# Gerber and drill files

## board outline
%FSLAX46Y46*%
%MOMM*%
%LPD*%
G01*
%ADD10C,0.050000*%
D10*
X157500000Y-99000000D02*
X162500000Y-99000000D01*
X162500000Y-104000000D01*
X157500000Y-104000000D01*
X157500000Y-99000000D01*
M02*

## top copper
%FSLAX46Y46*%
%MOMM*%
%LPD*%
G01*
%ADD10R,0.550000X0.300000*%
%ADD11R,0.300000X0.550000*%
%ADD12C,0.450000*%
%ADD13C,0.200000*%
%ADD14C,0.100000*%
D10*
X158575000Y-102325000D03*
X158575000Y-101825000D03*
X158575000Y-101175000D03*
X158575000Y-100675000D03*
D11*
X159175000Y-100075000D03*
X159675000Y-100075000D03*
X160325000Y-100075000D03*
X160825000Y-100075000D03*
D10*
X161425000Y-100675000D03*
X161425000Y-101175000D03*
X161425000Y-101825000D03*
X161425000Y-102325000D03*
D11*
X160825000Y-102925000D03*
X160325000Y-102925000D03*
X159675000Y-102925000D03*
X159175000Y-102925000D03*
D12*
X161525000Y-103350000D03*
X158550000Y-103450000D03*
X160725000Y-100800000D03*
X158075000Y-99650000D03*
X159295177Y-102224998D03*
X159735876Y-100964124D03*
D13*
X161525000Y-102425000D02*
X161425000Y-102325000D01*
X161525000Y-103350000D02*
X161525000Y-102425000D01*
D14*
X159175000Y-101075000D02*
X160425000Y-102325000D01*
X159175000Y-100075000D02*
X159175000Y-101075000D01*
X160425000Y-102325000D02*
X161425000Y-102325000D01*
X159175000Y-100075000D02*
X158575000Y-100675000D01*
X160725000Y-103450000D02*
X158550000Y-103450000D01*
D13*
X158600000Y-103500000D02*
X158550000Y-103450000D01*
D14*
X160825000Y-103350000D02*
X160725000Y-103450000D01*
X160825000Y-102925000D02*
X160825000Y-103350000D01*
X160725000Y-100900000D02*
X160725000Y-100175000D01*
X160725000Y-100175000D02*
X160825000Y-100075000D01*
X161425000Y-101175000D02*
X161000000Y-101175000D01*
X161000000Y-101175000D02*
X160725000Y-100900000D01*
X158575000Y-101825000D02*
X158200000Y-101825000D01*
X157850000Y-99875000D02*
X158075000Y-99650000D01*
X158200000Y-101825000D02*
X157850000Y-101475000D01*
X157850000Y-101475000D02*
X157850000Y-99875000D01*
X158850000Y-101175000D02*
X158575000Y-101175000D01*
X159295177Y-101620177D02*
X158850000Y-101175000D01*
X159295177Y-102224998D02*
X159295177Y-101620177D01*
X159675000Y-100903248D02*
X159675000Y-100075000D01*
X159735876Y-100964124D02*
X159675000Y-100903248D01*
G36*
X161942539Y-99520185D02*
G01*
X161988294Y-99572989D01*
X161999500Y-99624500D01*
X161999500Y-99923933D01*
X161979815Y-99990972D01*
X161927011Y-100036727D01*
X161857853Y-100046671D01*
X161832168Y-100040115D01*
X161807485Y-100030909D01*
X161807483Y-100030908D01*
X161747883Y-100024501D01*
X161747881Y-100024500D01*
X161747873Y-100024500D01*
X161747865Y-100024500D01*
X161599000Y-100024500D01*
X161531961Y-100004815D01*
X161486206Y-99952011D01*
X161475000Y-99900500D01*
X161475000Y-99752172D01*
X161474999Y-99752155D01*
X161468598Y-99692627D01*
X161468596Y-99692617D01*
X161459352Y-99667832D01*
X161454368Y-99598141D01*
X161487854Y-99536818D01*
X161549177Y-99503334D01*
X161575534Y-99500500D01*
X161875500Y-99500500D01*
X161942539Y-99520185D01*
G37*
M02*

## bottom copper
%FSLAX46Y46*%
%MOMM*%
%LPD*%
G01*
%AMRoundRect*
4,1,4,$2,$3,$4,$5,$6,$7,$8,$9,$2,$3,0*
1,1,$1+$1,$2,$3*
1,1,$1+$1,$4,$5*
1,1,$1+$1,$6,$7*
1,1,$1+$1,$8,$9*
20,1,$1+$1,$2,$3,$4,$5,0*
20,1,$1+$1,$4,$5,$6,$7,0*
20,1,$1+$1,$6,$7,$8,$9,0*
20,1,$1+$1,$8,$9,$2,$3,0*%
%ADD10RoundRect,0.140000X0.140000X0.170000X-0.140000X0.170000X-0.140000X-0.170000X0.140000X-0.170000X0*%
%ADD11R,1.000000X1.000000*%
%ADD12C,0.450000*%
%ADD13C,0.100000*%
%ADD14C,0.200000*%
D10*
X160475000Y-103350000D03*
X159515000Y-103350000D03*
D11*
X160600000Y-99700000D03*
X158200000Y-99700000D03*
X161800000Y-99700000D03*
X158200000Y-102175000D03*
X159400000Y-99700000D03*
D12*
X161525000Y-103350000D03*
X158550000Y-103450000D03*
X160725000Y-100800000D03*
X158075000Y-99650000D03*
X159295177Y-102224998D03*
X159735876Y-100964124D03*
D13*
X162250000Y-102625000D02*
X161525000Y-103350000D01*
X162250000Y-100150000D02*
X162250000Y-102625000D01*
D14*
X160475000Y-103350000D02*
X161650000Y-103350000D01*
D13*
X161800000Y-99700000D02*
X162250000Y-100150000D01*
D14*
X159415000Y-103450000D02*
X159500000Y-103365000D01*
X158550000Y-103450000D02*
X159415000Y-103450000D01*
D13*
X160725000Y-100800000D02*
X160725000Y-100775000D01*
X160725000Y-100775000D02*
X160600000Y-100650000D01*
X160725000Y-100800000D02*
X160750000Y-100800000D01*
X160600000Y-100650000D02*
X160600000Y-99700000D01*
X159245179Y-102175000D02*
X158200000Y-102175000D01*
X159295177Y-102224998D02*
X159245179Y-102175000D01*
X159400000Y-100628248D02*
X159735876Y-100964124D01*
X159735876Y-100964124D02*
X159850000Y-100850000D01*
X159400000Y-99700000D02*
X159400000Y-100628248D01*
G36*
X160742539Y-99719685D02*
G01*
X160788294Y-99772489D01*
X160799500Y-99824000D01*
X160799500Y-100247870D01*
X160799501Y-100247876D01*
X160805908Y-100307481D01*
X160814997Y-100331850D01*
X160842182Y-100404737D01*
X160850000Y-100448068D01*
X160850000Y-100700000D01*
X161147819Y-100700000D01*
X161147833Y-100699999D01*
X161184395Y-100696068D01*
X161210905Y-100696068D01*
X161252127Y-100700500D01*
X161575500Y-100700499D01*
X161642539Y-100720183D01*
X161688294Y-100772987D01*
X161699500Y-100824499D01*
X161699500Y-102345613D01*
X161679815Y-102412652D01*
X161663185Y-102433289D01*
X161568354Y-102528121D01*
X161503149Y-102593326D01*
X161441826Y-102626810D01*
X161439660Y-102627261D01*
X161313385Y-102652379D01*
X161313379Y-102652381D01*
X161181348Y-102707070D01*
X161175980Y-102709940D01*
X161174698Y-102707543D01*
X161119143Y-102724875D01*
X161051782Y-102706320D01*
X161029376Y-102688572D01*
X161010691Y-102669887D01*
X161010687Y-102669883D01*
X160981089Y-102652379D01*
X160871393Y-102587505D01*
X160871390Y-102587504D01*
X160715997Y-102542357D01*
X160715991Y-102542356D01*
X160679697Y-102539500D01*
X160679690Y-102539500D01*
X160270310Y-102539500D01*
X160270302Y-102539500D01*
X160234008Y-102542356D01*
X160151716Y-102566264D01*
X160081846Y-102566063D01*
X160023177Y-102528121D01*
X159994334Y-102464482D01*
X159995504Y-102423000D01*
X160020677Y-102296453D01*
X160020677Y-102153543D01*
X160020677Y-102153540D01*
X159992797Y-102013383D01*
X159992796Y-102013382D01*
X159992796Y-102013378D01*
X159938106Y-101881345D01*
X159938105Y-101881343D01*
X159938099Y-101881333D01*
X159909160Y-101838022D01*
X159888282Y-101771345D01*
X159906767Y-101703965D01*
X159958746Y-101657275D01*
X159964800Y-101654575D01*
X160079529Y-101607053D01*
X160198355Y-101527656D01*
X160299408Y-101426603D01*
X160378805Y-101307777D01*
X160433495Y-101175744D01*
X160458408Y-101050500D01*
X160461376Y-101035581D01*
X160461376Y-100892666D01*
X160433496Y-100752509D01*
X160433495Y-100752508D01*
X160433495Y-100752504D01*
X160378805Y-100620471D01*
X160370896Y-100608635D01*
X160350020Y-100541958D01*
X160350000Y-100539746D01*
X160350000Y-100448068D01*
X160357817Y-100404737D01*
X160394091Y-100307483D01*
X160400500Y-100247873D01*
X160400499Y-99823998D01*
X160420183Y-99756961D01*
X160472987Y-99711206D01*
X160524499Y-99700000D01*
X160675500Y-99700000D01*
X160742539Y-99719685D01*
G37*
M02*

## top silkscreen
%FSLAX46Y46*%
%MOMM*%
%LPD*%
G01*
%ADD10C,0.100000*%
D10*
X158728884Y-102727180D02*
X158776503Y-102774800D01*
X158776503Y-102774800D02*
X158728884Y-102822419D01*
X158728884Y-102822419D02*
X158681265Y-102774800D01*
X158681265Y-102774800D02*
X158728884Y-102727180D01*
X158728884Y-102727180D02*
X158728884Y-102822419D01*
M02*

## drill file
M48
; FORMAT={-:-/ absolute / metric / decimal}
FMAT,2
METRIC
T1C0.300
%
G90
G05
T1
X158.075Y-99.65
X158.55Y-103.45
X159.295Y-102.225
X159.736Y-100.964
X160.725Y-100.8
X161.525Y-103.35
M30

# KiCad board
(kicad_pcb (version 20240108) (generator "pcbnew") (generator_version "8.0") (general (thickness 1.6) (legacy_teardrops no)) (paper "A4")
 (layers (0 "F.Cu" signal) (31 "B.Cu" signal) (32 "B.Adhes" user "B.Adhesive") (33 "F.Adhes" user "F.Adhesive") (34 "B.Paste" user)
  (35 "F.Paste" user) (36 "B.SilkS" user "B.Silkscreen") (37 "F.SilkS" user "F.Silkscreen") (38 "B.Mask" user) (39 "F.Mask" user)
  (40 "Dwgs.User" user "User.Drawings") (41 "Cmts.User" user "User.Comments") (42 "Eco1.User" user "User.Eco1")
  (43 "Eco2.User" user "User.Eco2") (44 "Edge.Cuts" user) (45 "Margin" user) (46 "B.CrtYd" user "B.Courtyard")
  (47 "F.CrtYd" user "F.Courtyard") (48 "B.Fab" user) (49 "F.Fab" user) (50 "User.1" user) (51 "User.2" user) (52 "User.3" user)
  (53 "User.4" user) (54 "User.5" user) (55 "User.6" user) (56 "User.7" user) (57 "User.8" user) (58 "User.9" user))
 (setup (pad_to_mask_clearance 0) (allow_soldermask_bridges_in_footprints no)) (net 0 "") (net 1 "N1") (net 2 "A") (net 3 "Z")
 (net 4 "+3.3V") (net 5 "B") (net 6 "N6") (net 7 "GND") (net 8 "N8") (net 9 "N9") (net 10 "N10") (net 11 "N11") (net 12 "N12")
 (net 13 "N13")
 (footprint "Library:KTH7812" (layer "F.Cu") (at 158.5 103)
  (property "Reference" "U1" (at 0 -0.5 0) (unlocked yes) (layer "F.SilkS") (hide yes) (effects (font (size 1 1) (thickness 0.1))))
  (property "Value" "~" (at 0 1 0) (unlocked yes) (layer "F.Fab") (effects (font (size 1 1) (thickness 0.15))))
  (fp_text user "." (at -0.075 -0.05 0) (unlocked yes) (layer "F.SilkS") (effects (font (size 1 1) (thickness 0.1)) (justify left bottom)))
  (pad "1" smd rect (at 0.075 -0.675 180) (size 0.55 0.3) (layers "F.Cu" "F.Paste" "F.Mask") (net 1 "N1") (thermal_bridge_angle 45))
  (pad "2" smd rect (at 0.075 -1.175 180) (size 0.55 0.3) (layers "F.Cu" "F.Paste" "F.Mask") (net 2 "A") (thermal_bridge_angle 45))
  (pad "3" smd rect (at 0.075 -1.825 180) (size 0.55 0.3) (layers "F.Cu" "F.Paste" "F.Mask") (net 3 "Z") (thermal_bridge_angle 45))
  (pad "4" smd rect (at 0.075 -2.325 180) (size 0.55 0.3) (layers "F.Cu" "F.Paste" "F.Mask") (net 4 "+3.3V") (thermal_bridge_angle 45))
  (pad "5" smd rect (at 0.675 -2.925 90) (size 0.55 0.3) (layers "F.Cu" "F.Paste" "F.Mask") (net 4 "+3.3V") (thermal_bridge_angle 45))
  (pad "6" smd rect (at 1.175 -2.925 90) (size 0.55 0.3) (layers "F.Cu" "F.Paste" "F.Mask") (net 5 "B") (thermal_bridge_angle 45))
  (pad "7" smd rect (at 1.825 -2.925 90) (size 0.55 0.3) (layers "F.Cu" "F.Paste" "F.Mask") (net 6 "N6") (thermal_bridge_angle 45))
  (pad "8" smd rect (at 2.325 -2.925 90) (size 0.55 0.3) (layers "F.Cu" "F.Paste" "F.Mask") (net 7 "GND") (thermal_bridge_angle 45))
  (pad "9" smd rect (at 2.925 -2.325) (size 0.55 0.3) (layers "F.Cu" "F.Paste" "F.Mask") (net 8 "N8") (thermal_bridge_angle 45))
  (pad "10" smd rect (at 2.925 -1.825) (size 0.55 0.3) (layers "F.Cu" "F.Paste" "F.Mask") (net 7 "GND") (thermal_bridge_angle 45))
  (pad "11" smd rect (at 2.925 -1.175) (size 0.55 0.3) (layers "F.Cu" "F.Paste" "F.Mask") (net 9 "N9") (thermal_bridge_angle 45))
  (pad "12" smd rect (at 2.925 -0.675) (size 0.55 0.3) (layers "F.Cu" "F.Paste" "F.Mask") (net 4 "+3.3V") (thermal_bridge_angle 45))
  (pad "13" smd rect (at 2.325 -0.075 270) (size 0.55 0.3) (layers "F.Cu" "F.Paste" "F.Mask") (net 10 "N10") (thermal_bridge_angle 45))
  (pad "14" smd rect (at 1.825 -0.075 270) (size 0.55 0.3) (layers "F.Cu" "F.Paste" "F.Mask") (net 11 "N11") (thermal_bridge_angle 45))
  (pad "15" smd rect (at 1.175 -0.075 270) (size 0.55 0.3) (layers "F.Cu" "F.Paste" "F.Mask") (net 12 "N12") (thermal_bridge_angle 45))
  (pad "16" smd rect (at 0.675 -0.075 270) (size 0.55 0.3) (layers "F.Cu" "F.Paste" "F.Mask") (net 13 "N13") (thermal_bridge_angle 45)))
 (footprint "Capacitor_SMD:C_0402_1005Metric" (layer "B.Cu") (at 159.995 103.35 180)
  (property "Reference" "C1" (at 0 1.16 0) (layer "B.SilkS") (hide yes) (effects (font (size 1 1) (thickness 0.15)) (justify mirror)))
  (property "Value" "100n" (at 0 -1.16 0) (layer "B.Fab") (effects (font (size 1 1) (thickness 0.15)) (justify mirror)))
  (pad "1" smd roundrect (at -0.48 0 180) (size 0.56 0.62) (layers "B.Cu" "B.Paste" "B.Mask") (roundrect_rratio 0.25) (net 4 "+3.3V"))
  (pad "2" smd roundrect (at 0.48 0 180) (size 0.56 0.62) (layers "B.Cu" "B.Paste" "B.Mask") (roundrect_rratio 0.25) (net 10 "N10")))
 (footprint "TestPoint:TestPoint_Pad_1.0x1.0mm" (layer "B.Cu") (at 160.6 99.7 180)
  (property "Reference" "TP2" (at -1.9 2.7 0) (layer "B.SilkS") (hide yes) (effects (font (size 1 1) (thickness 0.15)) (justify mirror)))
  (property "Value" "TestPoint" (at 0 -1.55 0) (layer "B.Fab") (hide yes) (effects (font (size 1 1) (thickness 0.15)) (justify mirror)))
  (pad "1" smd rect (at 0 0 180) (size 1 1) (layers "B.Cu" "B.Mask") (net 7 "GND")))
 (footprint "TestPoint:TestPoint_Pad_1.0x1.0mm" (layer "B.Cu") (at 158.2 99.7 180)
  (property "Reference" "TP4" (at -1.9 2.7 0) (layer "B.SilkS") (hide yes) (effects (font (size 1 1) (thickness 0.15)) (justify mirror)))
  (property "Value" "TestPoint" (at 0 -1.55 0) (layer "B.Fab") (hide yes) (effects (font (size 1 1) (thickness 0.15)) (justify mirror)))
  (pad "1" smd rect (at 0 0 180) (size 1 1) (layers "B.Cu" "B.Mask") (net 2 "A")))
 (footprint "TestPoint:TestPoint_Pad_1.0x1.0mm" (layer "B.Cu") (at 161.8 99.7 180)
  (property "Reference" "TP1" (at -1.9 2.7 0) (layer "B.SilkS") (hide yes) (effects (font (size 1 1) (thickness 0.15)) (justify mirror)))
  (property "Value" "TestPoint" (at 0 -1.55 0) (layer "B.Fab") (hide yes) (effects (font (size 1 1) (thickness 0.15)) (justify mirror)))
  (pad "1" smd rect (at 0 0 180) (size 1 1) (layers "B.Cu" "B.Mask") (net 4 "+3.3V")))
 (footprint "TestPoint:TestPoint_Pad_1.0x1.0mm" (layer "B.Cu") (at 158.2 102.175 180)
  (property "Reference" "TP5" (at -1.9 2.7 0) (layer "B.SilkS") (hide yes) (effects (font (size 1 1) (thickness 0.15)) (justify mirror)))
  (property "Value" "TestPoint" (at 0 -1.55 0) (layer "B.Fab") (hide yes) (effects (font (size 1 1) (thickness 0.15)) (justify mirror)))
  (pad "1" smd rect (at 0 0 180) (size 1 1) (layers "B.Cu" "B.Mask") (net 3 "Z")))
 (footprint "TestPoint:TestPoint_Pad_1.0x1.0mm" (layer "B.Cu") (at 159.4 99.7 180)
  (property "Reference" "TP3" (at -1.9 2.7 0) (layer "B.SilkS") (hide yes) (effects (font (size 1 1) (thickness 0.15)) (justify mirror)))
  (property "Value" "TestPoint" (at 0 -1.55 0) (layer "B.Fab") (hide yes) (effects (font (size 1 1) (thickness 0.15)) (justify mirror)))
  (pad "1" smd rect (at 0 0 180) (size 1 1) (layers "B.Cu" "B.Mask") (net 5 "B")))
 (gr_rect (start 157.5 99) (end 162.5 104) (stroke (width 0.05) (type default)) (fill none) (layer "Edge.Cuts"))
 (segment (start 161.525 102.425) (end 161.425 102.325) (width 0.2) (layer "F.Cu") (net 4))
 (segment (start 161.525 103.35) (end 161.525 102.425) (width 0.2) (layer "F.Cu") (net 4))
 (segment (start 159.175 101.075) (end 160.425 102.325) (width 0.1) (layer "F.Cu") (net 4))
 (segment (start 159.175 100.075) (end 159.175 101.075) (width 0.1) (layer "F.Cu") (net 4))
 (segment (start 160.425 102.325) (end 161.425 102.325) (width 0.1) (layer "F.Cu") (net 4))
 (segment (start 159.175 100.075) (end 158.575 100.675) (width 0.1) (layer "F.Cu") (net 4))
 (via (at 161.525 103.35) (size 0.45) (drill 0.3) (layers "F.Cu" "B.Cu") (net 4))
 (segment (start 162.25 102.625) (end 161.525 103.35) (width 0.1) (layer "B.Cu") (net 4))
 (segment (start 162.25 100.15) (end 162.25 102.625) (width 0.1) (layer "B.Cu") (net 4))
 (segment (start 160.475 103.35) (end 161.65 103.35) (width 0.2) (layer "B.Cu") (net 4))
 (segment (start 161.8 99.7) (end 162.25 100.15) (width 0.1) (layer "B.Cu") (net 4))
 (segment (start 160.725 103.45) (end 158.55 103.45) (width 0.1) (layer "F.Cu") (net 10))
 (segment (start 158.6 103.5) (end 158.55 103.45) (width 0.2) (layer "F.Cu") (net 10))
 (segment (start 160.825 103.35) (end 160.725 103.45) (width 0.1) (layer "F.Cu") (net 10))
 (segment (start 160.825 102.925) (end 160.825 103.35) (width 0.1) (layer "F.Cu") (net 10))
 (via (at 158.55 103.45) (size 0.45) (drill 0.3) (layers "F.Cu" "B.Cu") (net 10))
 (segment (start 159.415 103.45) (end 159.5 103.365) (width 0.2) (layer "B.Cu") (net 10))
 (segment (start 158.55 103.45) (end 159.415 103.45) (width 0.2) (layer "B.Cu") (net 10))
 (segment (start 160.725 100.9) (end 160.725 100.175) (width 0.1) (layer "F.Cu") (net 7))
 (segment (start 160.725 100.175) (end 160.825 100.075) (width 0.1) (layer "F.Cu") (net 7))
 (segment (start 161.425 101.175) (end 161 101.175) (width 0.1) (layer "F.Cu") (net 7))
 (segment (start 161 101.175) (end 160.725 100.9) (width 0.1) (layer "F.Cu") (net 7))
 (via (at 160.725 100.8) (size 0.45) (drill 0.3) (layers "F.Cu" "B.Cu") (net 7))
 (segment (start 160.725 100.8) (end 160.725 100.775) (width 0.1) (layer "B.Cu") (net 7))
 (segment (start 160.725 100.775) (end 160.6 100.65) (width 0.1) (layer "B.Cu") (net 7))
 (segment (start 160.725 100.8) (end 160.75 100.8) (width 0.1) (layer "B.Cu") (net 7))
 (segment (start 160.6 100.65) (end 160.6 99.7) (width 0.1) (layer "B.Cu") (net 7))
 (segment (start 158.575 101.825) (end 158.2 101.825) (width 0.1) (layer "F.Cu") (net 2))
 (segment (start 157.85 99.875) (end 158.075 99.65) (width 0.1) (layer "F.Cu") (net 2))
 (segment (start 158.2 101.825) (end 157.85 101.475) (width 0.1) (layer "F.Cu") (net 2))
 (segment (start 157.85 101.475) (end 157.85 99.875) (width 0.1) (layer "F.Cu") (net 2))
 (via (at 158.075 99.65) (size 0.45) (drill 0.3) (layers "F.Cu" "B.Cu") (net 2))
 (segment (start 158.85 101.175) (end 158.575 101.175) (width 0.1) (layer "F.Cu") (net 3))
 (segment (start 159.295177 101.620177) (end 158.85 101.175) (width 0.1) (layer "F.Cu") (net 3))
 (segment (start 159.295177 102.224998) (end 159.295177 101.620177) (width 0.1) (layer "F.Cu") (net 3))
 (via (at 159.295177 102.224998) (size 0.45) (drill 0.3) (layers "F.Cu" "B.Cu") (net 3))
 (segment (start 159.245179 102.175) (end 158.2 102.175) (width 0.1) (layer "B.Cu") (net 3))
 (segment (start 159.295177 102.224998) (end 159.245179 102.175) (width 0.1) (layer "B.Cu") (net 3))
 (segment (start 159.675 100.903248) (end 159.675 100.075) (width 0.1) (layer "F.Cu") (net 5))
 (segment (start 159.735876 100.964124) (end 159.675 100.903248) (width 0.1) (layer "F.Cu") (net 5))
 (via (at 159.735876 100.964124) (size 0.45) (drill 0.3) (layers "F.Cu" "B.Cu") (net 5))
 (segment (start 159.4 100.628248) (end 159.735876 100.964124) (width 0.1) (layer "B.Cu") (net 5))
 (segment (start 159.735876 100.964124) (end 159.85 100.85) (width 0.1) (layer "B.Cu") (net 5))
 (segment (start 159.4 99.7) (end 159.4 100.628248) (width 0.1) (layer "B.Cu") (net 5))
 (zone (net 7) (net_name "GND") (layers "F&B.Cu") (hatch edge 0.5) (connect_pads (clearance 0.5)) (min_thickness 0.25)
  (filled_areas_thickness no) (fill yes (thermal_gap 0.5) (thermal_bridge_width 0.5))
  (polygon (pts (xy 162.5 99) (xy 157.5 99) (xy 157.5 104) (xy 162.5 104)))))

